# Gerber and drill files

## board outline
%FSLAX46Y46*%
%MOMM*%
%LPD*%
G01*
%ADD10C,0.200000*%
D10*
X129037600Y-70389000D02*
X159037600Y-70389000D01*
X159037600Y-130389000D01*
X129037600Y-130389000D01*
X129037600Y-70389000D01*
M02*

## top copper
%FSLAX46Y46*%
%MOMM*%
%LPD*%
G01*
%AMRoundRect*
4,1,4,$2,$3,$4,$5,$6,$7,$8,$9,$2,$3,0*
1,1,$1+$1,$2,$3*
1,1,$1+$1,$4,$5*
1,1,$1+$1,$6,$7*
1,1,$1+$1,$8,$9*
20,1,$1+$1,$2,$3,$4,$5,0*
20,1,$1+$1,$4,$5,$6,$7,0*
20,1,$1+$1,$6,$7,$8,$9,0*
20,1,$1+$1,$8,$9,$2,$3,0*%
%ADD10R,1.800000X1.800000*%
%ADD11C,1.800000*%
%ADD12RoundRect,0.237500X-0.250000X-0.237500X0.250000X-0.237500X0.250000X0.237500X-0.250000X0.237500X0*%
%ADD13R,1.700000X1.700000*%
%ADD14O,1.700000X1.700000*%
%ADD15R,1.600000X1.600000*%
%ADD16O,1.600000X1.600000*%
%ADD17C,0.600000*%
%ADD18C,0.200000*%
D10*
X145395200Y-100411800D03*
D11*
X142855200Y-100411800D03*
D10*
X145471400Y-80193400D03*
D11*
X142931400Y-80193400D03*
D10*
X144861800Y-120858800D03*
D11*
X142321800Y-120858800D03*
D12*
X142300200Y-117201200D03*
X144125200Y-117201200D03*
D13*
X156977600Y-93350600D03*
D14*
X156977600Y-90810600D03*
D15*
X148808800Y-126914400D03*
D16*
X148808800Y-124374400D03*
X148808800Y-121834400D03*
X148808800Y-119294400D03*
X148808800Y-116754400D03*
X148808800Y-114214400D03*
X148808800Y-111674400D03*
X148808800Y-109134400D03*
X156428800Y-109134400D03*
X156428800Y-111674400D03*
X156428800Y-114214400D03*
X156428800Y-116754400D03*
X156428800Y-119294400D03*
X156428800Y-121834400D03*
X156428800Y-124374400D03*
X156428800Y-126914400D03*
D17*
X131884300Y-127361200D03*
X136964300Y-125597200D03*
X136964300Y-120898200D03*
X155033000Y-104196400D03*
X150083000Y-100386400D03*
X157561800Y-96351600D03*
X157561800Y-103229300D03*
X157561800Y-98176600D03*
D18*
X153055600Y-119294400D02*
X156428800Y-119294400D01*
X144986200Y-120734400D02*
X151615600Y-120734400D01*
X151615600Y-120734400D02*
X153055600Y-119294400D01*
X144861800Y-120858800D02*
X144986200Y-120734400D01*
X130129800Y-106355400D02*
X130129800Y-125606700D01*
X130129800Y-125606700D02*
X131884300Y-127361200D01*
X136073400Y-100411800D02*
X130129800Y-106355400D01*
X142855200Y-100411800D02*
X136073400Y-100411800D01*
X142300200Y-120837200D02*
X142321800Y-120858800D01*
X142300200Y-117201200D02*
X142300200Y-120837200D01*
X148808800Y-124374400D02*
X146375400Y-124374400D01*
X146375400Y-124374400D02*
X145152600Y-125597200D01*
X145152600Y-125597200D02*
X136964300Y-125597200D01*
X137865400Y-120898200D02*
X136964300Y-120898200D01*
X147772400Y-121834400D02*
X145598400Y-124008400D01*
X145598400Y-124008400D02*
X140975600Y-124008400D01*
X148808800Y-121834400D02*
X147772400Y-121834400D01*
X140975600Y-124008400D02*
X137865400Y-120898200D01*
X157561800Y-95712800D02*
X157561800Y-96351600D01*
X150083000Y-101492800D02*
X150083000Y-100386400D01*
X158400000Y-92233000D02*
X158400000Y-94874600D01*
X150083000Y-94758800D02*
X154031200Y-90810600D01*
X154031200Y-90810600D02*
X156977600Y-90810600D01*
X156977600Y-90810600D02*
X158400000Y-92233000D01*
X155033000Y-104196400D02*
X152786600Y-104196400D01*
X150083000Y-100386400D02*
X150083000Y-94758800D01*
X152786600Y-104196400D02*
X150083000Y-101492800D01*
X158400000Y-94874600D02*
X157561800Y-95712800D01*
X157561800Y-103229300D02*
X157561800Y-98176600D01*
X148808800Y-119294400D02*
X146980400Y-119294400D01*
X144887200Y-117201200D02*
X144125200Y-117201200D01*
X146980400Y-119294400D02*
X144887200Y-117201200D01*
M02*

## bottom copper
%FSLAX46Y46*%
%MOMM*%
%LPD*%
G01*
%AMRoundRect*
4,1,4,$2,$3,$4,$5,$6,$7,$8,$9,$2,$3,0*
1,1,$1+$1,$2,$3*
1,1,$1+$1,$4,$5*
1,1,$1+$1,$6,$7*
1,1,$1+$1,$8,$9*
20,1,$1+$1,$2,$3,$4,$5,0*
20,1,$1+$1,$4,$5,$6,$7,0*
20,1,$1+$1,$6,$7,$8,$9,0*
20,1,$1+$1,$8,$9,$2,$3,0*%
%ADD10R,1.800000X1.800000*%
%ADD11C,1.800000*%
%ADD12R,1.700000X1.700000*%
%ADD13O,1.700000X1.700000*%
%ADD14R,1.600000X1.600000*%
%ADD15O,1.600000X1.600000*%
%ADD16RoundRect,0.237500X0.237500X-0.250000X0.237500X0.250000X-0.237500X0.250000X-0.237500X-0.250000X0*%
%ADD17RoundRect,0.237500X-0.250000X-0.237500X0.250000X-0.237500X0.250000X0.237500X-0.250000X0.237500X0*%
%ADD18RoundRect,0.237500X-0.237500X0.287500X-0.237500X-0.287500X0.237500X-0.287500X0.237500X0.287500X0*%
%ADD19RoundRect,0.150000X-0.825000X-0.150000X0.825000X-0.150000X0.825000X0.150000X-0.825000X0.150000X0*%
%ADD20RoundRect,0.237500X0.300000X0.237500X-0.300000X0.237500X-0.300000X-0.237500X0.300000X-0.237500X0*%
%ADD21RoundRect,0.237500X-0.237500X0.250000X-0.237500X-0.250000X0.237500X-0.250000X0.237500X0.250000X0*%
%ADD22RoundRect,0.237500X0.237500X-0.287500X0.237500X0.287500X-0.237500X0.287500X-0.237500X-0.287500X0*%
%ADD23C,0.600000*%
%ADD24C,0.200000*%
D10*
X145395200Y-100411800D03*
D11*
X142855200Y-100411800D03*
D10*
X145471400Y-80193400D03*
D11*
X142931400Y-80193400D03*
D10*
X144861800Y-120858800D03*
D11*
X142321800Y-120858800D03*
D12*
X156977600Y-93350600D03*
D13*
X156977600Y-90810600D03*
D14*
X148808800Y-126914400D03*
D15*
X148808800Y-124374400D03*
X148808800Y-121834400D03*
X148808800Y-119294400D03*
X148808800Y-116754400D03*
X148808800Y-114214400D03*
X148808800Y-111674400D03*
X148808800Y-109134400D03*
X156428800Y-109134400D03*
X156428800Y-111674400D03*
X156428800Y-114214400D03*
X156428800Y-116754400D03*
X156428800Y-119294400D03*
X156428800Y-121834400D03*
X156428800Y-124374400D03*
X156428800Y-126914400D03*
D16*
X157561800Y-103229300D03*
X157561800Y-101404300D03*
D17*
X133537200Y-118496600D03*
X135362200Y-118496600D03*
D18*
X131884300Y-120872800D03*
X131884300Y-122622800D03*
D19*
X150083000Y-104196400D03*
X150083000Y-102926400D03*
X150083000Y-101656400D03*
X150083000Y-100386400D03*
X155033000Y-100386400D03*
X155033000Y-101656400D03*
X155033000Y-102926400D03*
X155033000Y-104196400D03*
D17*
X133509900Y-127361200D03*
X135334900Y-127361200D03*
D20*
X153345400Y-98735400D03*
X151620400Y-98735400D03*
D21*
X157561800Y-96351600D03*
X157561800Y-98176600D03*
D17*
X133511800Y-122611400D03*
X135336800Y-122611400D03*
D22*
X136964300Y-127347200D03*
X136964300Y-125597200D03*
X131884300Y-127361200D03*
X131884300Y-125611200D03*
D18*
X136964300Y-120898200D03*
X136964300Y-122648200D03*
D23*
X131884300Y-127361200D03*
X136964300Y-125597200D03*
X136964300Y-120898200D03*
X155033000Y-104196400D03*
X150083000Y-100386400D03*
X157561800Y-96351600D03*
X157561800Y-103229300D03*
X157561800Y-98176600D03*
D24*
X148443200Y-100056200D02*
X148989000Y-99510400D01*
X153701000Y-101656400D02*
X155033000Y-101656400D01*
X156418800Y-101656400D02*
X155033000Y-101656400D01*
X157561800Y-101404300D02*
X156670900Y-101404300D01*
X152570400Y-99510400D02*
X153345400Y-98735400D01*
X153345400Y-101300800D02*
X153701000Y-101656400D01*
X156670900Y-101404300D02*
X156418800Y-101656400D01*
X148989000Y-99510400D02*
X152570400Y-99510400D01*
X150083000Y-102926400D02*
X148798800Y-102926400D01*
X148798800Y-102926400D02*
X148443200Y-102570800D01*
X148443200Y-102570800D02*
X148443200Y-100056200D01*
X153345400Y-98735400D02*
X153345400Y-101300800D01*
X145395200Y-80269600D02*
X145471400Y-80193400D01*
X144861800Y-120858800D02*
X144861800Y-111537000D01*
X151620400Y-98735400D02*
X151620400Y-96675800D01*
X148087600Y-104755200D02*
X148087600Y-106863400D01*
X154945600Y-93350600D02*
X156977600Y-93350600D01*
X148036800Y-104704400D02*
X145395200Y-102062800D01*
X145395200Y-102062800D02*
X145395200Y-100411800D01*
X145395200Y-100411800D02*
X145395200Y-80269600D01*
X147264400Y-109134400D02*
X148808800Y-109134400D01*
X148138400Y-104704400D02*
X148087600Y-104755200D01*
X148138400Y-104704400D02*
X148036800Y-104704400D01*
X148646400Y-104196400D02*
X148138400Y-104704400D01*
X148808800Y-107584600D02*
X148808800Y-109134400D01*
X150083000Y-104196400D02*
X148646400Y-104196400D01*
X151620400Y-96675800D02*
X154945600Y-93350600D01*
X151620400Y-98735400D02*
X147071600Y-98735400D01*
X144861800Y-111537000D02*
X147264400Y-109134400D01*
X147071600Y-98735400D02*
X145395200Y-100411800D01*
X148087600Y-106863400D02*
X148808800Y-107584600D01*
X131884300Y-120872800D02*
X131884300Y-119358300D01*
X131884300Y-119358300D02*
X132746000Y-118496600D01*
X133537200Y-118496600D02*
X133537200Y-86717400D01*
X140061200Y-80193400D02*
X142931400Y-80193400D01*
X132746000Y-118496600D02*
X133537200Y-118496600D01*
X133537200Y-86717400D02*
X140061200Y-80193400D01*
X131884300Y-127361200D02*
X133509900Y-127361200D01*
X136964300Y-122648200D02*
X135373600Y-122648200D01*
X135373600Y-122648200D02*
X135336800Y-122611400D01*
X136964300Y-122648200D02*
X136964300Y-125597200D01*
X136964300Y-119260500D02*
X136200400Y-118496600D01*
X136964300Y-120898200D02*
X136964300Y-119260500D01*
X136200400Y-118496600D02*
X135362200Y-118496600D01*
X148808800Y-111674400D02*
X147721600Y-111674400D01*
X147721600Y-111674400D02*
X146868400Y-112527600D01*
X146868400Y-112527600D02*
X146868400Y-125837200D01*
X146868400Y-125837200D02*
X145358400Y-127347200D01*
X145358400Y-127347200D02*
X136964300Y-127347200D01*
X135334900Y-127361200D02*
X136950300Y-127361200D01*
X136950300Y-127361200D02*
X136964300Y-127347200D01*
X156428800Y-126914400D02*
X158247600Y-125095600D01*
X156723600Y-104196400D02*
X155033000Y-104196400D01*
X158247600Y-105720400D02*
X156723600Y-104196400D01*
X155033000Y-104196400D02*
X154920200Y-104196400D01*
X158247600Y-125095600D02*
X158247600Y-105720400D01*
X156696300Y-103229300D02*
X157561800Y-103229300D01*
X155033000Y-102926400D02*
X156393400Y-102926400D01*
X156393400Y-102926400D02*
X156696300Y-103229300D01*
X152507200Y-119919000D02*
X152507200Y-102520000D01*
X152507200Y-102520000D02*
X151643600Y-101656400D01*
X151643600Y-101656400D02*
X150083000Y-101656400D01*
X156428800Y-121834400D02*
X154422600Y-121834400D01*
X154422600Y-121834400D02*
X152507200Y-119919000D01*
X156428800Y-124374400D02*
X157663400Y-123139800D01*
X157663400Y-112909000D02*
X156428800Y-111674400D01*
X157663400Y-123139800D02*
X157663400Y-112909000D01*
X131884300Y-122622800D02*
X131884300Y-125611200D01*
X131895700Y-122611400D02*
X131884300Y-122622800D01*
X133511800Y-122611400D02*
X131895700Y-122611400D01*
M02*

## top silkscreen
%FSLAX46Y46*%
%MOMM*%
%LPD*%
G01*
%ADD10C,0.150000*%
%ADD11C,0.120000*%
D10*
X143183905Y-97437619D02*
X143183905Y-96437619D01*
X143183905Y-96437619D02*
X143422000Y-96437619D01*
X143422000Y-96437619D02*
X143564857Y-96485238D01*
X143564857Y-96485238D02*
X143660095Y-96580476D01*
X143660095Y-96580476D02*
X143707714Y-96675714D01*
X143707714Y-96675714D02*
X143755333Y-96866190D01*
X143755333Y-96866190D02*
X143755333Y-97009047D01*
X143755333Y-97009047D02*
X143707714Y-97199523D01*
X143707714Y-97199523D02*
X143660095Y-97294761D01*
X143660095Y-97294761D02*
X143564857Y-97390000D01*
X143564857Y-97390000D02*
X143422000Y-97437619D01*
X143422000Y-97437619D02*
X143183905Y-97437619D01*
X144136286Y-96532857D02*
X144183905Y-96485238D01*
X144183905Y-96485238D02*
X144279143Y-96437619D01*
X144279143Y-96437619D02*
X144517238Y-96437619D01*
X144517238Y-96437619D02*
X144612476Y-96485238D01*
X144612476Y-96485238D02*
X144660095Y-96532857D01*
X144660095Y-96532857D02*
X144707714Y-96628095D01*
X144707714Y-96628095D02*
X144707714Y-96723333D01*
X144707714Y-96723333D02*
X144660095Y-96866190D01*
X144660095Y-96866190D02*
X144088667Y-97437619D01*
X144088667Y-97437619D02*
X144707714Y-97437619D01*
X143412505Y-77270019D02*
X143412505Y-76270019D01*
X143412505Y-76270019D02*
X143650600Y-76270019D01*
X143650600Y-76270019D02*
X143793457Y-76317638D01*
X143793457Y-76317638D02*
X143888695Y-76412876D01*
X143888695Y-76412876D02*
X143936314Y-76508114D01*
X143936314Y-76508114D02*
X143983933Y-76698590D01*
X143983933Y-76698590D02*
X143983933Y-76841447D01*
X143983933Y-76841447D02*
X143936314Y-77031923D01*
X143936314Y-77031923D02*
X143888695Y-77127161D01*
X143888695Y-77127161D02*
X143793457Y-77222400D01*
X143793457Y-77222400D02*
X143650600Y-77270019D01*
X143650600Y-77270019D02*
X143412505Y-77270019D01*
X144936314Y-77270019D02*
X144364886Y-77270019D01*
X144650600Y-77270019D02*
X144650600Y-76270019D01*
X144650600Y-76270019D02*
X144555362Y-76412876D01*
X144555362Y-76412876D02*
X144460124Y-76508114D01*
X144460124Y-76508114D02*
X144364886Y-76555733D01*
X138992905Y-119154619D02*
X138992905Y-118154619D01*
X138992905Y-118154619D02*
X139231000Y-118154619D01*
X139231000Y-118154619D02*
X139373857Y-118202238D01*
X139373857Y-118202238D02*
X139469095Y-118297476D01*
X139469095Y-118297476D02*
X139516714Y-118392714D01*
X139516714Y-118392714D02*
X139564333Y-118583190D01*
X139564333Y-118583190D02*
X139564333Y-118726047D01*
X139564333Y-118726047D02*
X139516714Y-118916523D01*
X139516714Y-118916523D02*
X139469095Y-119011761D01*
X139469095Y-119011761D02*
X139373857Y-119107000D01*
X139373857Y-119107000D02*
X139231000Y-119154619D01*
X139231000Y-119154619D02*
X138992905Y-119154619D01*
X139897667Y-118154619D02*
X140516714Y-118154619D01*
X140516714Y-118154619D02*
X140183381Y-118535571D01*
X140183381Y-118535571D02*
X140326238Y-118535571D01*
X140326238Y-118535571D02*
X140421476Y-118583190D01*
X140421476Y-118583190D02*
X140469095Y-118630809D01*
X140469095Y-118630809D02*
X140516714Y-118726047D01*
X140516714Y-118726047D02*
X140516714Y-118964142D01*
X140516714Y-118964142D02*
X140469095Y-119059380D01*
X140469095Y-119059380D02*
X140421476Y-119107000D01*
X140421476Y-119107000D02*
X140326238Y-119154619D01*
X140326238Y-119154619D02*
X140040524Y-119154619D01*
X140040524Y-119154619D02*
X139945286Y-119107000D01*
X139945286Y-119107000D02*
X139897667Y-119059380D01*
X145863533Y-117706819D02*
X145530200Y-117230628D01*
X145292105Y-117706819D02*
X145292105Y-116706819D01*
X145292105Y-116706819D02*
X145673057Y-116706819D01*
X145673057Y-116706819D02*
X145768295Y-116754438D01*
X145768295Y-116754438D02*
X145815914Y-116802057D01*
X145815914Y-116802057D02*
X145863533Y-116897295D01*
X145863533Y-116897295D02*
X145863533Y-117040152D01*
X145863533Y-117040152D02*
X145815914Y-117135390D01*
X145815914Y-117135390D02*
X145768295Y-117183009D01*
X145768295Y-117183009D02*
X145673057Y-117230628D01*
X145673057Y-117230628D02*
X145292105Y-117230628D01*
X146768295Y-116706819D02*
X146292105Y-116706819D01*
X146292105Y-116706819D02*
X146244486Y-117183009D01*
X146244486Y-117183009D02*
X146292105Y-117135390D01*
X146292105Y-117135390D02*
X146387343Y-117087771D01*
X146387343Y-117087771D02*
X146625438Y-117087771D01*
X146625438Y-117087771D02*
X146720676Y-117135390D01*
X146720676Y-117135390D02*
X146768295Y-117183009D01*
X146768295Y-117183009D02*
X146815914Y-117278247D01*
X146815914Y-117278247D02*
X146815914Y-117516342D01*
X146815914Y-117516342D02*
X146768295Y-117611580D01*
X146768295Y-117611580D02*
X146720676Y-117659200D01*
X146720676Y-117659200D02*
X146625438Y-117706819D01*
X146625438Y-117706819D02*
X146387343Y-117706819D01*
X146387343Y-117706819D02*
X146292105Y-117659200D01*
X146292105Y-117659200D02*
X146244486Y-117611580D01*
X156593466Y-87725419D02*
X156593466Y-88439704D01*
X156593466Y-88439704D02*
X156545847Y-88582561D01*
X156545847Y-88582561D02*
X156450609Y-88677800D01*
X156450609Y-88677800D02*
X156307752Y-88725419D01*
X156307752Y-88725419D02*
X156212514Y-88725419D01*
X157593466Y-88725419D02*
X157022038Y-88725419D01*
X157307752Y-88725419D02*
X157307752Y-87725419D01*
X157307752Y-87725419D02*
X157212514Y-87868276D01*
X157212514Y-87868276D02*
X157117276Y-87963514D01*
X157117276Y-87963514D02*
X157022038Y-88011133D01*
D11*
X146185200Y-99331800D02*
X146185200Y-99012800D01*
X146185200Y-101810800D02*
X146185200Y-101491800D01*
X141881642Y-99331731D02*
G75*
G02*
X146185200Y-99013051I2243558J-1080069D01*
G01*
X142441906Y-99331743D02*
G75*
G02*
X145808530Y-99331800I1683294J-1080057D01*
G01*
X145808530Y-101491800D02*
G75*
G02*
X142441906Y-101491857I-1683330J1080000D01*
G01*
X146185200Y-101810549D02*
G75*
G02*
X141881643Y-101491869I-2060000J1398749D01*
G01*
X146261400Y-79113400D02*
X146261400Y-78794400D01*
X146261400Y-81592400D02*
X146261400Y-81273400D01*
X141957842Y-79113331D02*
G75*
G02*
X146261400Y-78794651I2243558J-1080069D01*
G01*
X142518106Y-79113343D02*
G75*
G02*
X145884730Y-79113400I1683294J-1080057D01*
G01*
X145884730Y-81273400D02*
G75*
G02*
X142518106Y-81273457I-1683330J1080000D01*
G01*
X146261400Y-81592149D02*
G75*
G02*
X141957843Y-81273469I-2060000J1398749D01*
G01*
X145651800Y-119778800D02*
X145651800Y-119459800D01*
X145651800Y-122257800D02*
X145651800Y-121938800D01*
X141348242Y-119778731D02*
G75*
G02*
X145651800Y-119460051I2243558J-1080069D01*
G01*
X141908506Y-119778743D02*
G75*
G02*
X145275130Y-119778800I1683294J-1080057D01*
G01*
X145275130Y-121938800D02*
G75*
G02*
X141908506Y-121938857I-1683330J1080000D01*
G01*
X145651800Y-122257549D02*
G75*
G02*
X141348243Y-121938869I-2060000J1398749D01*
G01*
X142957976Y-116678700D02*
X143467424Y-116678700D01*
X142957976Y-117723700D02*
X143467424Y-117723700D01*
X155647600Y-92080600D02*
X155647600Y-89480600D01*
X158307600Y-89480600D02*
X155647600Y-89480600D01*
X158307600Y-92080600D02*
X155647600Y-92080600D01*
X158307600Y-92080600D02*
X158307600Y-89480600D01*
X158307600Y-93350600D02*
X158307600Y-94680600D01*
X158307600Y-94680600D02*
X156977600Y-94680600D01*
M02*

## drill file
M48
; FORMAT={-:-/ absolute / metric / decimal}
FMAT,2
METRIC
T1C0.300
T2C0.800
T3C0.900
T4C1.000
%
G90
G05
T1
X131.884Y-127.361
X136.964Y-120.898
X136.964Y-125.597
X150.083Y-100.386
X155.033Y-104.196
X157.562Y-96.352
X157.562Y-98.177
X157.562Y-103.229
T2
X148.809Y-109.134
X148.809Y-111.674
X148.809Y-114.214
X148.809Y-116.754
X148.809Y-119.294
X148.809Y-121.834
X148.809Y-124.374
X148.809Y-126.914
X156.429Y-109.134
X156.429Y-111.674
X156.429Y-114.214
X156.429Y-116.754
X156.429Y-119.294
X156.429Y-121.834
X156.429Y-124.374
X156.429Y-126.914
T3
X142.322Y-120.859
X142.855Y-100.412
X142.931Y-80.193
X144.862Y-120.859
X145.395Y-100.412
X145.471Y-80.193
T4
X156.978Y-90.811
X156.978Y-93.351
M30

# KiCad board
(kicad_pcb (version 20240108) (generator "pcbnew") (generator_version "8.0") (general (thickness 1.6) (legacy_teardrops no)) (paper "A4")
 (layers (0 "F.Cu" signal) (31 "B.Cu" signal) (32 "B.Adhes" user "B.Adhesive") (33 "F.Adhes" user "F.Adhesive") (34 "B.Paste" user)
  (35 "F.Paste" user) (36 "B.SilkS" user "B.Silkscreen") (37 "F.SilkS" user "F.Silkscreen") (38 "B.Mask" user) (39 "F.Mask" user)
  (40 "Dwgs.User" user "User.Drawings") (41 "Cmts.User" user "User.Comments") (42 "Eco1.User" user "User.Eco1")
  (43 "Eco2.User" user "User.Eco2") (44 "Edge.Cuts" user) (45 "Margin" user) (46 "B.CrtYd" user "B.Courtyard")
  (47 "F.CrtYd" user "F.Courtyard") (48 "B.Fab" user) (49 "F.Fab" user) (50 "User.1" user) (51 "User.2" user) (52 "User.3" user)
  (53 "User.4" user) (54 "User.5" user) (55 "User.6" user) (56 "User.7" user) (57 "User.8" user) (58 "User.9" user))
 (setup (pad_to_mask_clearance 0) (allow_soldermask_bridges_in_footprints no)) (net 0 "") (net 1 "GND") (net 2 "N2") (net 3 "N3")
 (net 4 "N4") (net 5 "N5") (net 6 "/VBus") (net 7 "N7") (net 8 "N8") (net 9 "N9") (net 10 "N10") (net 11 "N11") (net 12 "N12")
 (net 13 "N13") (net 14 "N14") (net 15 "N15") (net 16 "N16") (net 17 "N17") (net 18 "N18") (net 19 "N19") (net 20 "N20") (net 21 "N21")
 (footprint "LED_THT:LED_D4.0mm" (layer "F.Cu") (at 145.3952 100.4118 180)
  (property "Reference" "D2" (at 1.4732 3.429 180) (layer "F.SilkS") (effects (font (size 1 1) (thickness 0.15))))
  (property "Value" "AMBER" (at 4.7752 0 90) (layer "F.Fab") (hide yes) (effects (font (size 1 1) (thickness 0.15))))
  (fp_line (start -0.79 1.08) (end -0.79 1.399) (stroke (width 0.12) (type solid)) (layer "F.SilkS"))
  (fp_line (start -0.79 -1.399) (end -0.79 -1.08) (stroke (width 0.12) (type solid)) (layer "F.SilkS"))
  (fp_arc (start 3.513558 1.080069) (mid 1.453882 2.483201) (end -0.79 1.398749) (stroke (width 0.12) (type solid)) (layer "F.SilkS"))
  (fp_arc (start 2.953294 1.080057) (mid 1.269966 2) (end -0.41333 1.08) (stroke (width 0.12) (type solid)) (layer "F.SilkS"))
  (fp_arc (start -0.41333 -1.08) (mid 1.269966 -2) (end 2.953294 -1.080057) (stroke (width 0.12) (type solid)) (layer "F.SilkS"))
  (fp_arc (start -0.79 -1.398749) (mid 1.453882 -2.483201) (end 3.513558 -1.080069) (stroke (width 0.12) (type solid)) (layer "F.SilkS"))
  (pad "1" thru_hole rect (at 0 0 180) (size 1.8 1.8) (drill 0.9) (layers "*.Cu" "*.Mask") (remove_unused_layers no) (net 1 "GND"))
  (pad "2" thru_hole circle (at 2.54 0 180) (size 1.8 1.8) (drill 0.9) (layers "*.Cu" "*.Mask") (remove_unused_layers no) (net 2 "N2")))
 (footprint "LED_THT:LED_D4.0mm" (layer "F.Cu") (at 145.4714 80.1934 180)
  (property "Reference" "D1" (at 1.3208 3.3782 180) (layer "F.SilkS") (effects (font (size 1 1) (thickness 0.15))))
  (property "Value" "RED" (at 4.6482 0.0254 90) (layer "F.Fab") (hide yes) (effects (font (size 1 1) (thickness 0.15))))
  (fp_line (start -0.79 1.08) (end -0.79 1.399) (stroke (width 0.12) (type solid)) (layer "F.SilkS"))
  (fp_line (start -0.79 -1.399) (end -0.79 -1.08) (stroke (width 0.12) (type solid)) (layer "F.SilkS"))
  (fp_arc (start 3.513558 1.080069) (mid 1.453882 2.483201) (end -0.79 1.398749) (stroke (width 0.12) (type solid)) (layer "F.SilkS"))
  (fp_arc (start 2.953294 1.080057) (mid 1.269966 2) (end -0.41333 1.08) (stroke (width 0.12) (type solid)) (layer "F.SilkS"))
  (fp_arc (start -0.41333 -1.08) (mid 1.269966 -2) (end 2.953294 -1.080057) (stroke (width 0.12) (type solid)) (layer "F.SilkS"))
  (fp_arc (start -0.79 -1.398749) (mid 1.453882 -2.483201) (end 3.513558 -1.080069) (stroke (width 0.12) (type solid)) (layer "F.SilkS"))
  (pad "1" thru_hole rect (at 0 0 180) (size 1.8 1.8) (drill 0.9) (layers "*.Cu" "*.Mask") (remove_unused_layers no) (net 1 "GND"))
  (pad "2" thru_hole circle (at 2.54 0 180) (size 1.8 1.8) (drill 0.9) (layers "*.Cu" "*.Mask") (remove_unused_layers no) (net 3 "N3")))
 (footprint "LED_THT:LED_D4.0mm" (layer "F.Cu") (at 144.8618 120.8588 180)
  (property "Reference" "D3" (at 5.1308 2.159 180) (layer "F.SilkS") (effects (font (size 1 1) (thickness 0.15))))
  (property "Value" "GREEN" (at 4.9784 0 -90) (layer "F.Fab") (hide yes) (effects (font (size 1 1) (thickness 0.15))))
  (fp_line (start -0.79 1.08) (end -0.79 1.399) (stroke (width 0.12) (type solid)) (layer "F.SilkS"))
  (fp_line (start -0.79 -1.399) (end -0.79 -1.08) (stroke (width 0.12) (type solid)) (layer "F.SilkS"))
  (fp_arc (start 3.513558 1.080069) (mid 1.453882 2.483201) (end -0.79 1.398749) (stroke (width 0.12) (type solid)) (layer "F.SilkS"))
  (fp_arc (start 2.953294 1.080057) (mid 1.269966 2) (end -0.41333 1.08) (stroke (width 0.12) (type solid)) (layer "F.SilkS"))
  (fp_arc (start -0.41333 -1.08) (mid 1.269966 -2) (end 2.953294 -1.080057) (stroke (width 0.12) (type solid)) (layer "F.SilkS"))
  (fp_arc (start -0.79 -1.398749) (mid 1.453882 -2.483201) (end 3.513558 -1.080069) (stroke (width 0.12) (type solid)) (layer "F.SilkS"))
  (pad "1" thru_hole rect (at 0 0 180) (size 1.8 1.8) (drill 0.9) (layers "*.Cu" "*.Mask") (remove_unused_layers no) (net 1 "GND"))
  (pad "2" thru_hole circle (at 2.54 0 180) (size 1.8 1.8) (drill 0.9) (layers "*.Cu" "*.Mask") (remove_unused_layers no) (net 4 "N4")))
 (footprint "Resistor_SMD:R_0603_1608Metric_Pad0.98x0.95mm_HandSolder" (layer "F.Cu") (at 143.2127 117.2012)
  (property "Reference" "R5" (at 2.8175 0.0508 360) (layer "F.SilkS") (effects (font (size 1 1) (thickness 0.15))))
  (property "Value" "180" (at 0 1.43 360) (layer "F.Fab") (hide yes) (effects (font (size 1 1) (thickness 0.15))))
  (fp_line (start -0.254724 -0.5225) (end 0.254724 -0.5225) (stroke (width 0.12) (type solid)) (layer "F.SilkS"))
  (fp_line (start -0.254724 0.5225) (end 0.254724 0.5225) (stroke (width 0.12) (type solid)) (layer "F.SilkS"))
  (pad "1" smd roundrect (at -0.9125 0) (size 0.975 0.95) (layers "F.Cu" "F.Paste" "F.Mask") (roundrect_rratio 0.25) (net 4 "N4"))
  (pad "2" smd roundrect (at 0.9125 0) (size 0.975 0.95) (layers "F.Cu" "F.Paste" "F.Mask") (roundrect_rratio 0.25) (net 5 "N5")))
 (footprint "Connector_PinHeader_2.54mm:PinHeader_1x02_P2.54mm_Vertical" (layer "F.Cu") (at 156.9776 93.3506 180)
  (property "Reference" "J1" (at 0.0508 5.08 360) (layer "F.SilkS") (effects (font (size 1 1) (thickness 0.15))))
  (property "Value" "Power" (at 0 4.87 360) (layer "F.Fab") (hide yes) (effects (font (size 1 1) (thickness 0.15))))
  (fp_line (start 1.33 1.27) (end 1.33 3.87) (stroke (width 0.12) (type solid)) (layer "F.SilkS"))
  (fp_line (start -1.33 3.87) (end 1.33 3.87) (stroke (width 0.12) (type solid)) (layer "F.SilkS"))
  (fp_line (start -1.33 1.27) (end 1.33 1.27) (stroke (width 0.12) (type solid)) (layer "F.SilkS"))
  (fp_line (start -1.33 1.27) (end -1.33 3.87) (stroke (width 0.12) (type solid)) (layer "F.SilkS"))
  (fp_line (start -1.33 0) (end -1.33 -1.33) (stroke (width 0.12) (type solid)) (layer "F.SilkS"))
  (fp_line (start -1.33 -1.33) (end 0 -1.33) (stroke (width 0.12) (type solid)) (layer "F.SilkS"))
  (pad "1" thru_hole rect (at 0 0 180) (size 1.7 1.7) (drill 1) (layers "*.Cu" "*.Mask") (remove_unused_layers no) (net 1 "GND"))
  (pad "2" thru_hole oval (at 0 2.54 180) (size 1.7 1.7) (drill 1) (layers "*.Cu" "*.Mask") (remove_unused_layers no) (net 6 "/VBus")))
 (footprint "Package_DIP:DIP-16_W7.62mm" (layer "B.Cu") (at 148.8088 126.9144)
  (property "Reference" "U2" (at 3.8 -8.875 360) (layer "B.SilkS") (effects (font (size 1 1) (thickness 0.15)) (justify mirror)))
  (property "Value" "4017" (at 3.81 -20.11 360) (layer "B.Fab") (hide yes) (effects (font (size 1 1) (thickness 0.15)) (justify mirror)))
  (pad "1" thru_hole rect (at 0 0) (size 1.6 1.6) (drill 0.8) (layers "*.Cu" "*.Mask") (remove_unused_layers no) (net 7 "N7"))
  (pad "2" thru_hole oval (at 0 -2.54) (size 1.6 1.6) (drill 0.8) (layers "*.Cu" "*.Mask") (remove_unused_layers no) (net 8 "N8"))
  (pad "3" thru_hole oval (at 0 -5.08) (size 1.6 1.6) (drill 0.8) (layers "*.Cu" "*.Mask") (remove_unused_layers no) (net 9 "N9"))
  (pad "4" thru_hole oval (at 0 -7.62) (size 1.6 1.6) (drill 0.8) (layers "*.Cu" "*.Mask") (remove_unused_layers no) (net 5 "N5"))
  (pad "5" thru_hole oval (at 0 -10.16) (size 1.6 1.6) (drill 0.8) (layers "*.Cu" "*.Mask") (remove_unused_layers no) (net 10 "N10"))
  (pad "6" thru_hole oval (at 0 -12.7) (size 1.6 1.6) (drill 0.8) (layers "*.Cu" "*.Mask") (remove_unused_layers no) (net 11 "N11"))
  (pad "7" thru_hole oval (at 0 -15.24) (size 1.6 1.6) (drill 0.8) (layers "*.Cu" "*.Mask") (remove_unused_layers no) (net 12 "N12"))
  (pad "8" thru_hole oval (at 0 -17.78) (size 1.6 1.6) (drill 0.8) (layers "*.Cu" "*.Mask") (remove_unused_layers no) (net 1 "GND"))
  (pad "9" thru_hole oval (at 7.62 -17.78) (size 1.6 1.6) (drill 0.8) (layers "*.Cu" "*.Mask") (remove_unused_layers no) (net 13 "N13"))
  (pad "10" thru_hole oval (at 7.62 -15.24) (size 1.6 1.6) (drill 0.8) (layers "*.Cu" "*.Mask") (remove_unused_layers no) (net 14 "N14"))
  (pad "11" thru_hole oval (at 7.62 -12.7) (size 1.6 1.6) (drill 0.8) (layers "*.Cu" "*.Mask") (remove_unused_layers no) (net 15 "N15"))
  (pad "12" thru_hole oval (at 7.62 -10.16) (size 1.6 1.6) (drill 0.8) (layers "*.Cu" "*.Mask") (remove_unused_layers no) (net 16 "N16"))
  (pad "13" thru_hole oval (at 7.62 -7.62) (size 1.6 1.6) (drill 0.8) (layers "*.Cu" "*.Mask") (remove_unused_layers no) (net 1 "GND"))
  (pad "14" thru_hole oval (at 7.62 -5.08) (size 1.6 1.6) (drill 0.8) (layers "*.Cu" "*.Mask") (remove_unused_layers no) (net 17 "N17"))
  (pad "15" thru_hole oval (at 7.62 -2.54) (size 1.6 1.6) (drill 0.8) (layers "*.Cu" "*.Mask") (remove_unused_layers no) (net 14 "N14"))
  (pad "16" thru_hole oval (at 7.62 0) (size 1.6 1.6) (drill 0.8) (layers "*.Cu" "*.Mask") (remove_unused_layers no) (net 6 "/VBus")))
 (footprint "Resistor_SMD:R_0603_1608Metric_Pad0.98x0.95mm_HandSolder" (layer "B.Cu") (at 157.5618 102.3168 90)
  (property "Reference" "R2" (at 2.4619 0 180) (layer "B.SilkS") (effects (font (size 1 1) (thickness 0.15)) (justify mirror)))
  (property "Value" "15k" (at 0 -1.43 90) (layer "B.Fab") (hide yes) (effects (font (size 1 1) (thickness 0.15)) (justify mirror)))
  (pad "1" smd roundrect (at -0.9125 0 90) (size 0.975 0.95) (layers "B.Cu" "B.Paste" "B.Mask") (roundrect_rratio 0.25) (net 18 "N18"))
  (pad "2" smd roundrect (at 0.9125 0 90) (size 0.975 0.95) (layers "B.Cu" "B.Paste" "B.Mask") (roundrect_rratio 0.25) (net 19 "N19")))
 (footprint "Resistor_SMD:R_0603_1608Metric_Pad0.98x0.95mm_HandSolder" (layer "B.Cu") (at 134.4497 118.4966)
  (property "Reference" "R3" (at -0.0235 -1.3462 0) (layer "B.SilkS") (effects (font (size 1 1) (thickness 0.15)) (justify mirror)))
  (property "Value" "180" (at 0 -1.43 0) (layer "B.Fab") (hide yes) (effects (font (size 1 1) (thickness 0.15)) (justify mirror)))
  (pad "1" smd roundrect (at -0.9125 0) (size 0.975 0.95) (layers "B.Cu" "B.Paste" "B.Mask") (roundrect_rratio 0.25) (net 3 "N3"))
  (pad "2" smd roundrect (at 0.9125 0) (size 0.975 0.95) (layers "B.Cu" "B.Paste" "B.Mask") (roundrect_rratio 0.25) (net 9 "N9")))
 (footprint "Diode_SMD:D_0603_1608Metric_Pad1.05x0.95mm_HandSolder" (layer "B.Cu") (at 131.8843 121.7478 -90)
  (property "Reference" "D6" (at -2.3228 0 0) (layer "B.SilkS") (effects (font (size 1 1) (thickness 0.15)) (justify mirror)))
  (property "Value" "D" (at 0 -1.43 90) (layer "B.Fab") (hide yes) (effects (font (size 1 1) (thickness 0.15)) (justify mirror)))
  (pad "1" smd roundrect (at -0.875 0 270) (size 1.05 0.95) (layers "B.Cu" "B.Paste" "B.Mask") (roundrect_rratio 0.25) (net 3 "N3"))
  (pad "2" smd roundrect (at 0.875 0 270) (size 1.05 0.95) (layers "B.Cu" "B.Paste" "B.Mask") (roundrect_rratio 0.25) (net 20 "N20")))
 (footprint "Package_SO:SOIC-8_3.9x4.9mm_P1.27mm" (layer "B.Cu") (at 152.558 102.2914)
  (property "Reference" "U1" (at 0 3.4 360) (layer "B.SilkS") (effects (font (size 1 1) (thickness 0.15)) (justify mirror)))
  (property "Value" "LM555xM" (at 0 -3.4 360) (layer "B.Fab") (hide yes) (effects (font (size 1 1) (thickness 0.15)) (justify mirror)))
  (pad "1" smd roundrect (at -2.475 1.905) (size 1.95 0.6) (layers "B.Cu" "B.Paste" "B.Mask") (roundrect_rratio 0.25) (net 1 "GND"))
  (pad "2" smd roundrect (at -2.475 0.635) (size 1.95 0.6) (layers "B.Cu" "B.Paste" "B.Mask") (roundrect_rratio 0.25) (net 19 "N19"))
  (pad "3" smd roundrect (at -2.475 -0.635) (size 1.95 0.6) (layers "B.Cu" "B.Paste" "B.Mask") (roundrect_rratio 0.25) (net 17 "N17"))
  (pad "4" smd roundrect (at -2.475 -1.905) (size 1.95 0.6) (layers "B.Cu" "B.Paste" "B.Mask") (roundrect_rratio 0.25) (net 6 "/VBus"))
  (pad "5" smd roundrect (at 2.475 -1.905) (size 1.95 0.6) (layers "B.Cu" "B.Paste" "B.Mask") (roundrect_rratio 0.25) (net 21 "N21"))
  (pad "6" smd roundrect (at 2.475 -0.635) (size 1.95 0.6) (layers "B.Cu" "B.Paste" "B.Mask") (roundrect_rratio 0.25) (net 19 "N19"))
  (pad "7" smd roundrect (at 2.475 0.635) (size 1.95 0.6) (layers "B.Cu" "B.Paste" "B.Mask") (roundrect_rratio 0.25) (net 18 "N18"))
  (pad "8" smd roundrect (at 2.475 1.905) (size 1.95 0.6) (layers "B.Cu" "B.Paste" "B.Mask") (roundrect_rratio 0.25) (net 6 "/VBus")))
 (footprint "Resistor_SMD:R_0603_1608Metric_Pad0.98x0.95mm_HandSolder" (layer "B.Cu") (at 134.4224 127.3612)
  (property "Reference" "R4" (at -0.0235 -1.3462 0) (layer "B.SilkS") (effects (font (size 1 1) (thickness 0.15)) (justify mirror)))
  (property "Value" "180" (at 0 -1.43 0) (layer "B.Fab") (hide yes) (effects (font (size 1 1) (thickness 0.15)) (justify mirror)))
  (pad "1" smd roundrect (at -0.9125 0) (size 0.975 0.95) (layers "B.Cu" "B.Paste" "B.Mask") (roundrect_rratio 0.25) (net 2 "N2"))
  (pad "2" smd roundrect (at 0.9125 0) (size 0.975 0.95) (layers "B.Cu" "B.Paste" "B.Mask") (roundrect_rratio 0.25) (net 12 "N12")))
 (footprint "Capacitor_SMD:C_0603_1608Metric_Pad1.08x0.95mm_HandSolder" (layer "B.Cu") (at 152.4829 98.7354 180)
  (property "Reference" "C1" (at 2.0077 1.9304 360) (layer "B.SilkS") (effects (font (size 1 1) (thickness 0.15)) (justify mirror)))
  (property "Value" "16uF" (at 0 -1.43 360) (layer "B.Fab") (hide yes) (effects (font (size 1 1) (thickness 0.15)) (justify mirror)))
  (pad "1" smd roundrect (at -0.8625 0 180) (size 1.075 0.95) (layers "B.Cu" "B.Paste" "B.Mask") (roundrect_rratio 0.25) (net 19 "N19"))
  (pad "2" smd roundrect (at 0.8625 0 180) (size 1.075 0.95) (layers "B.Cu" "B.Paste" "B.Mask") (roundrect_rratio 0.25) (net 1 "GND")))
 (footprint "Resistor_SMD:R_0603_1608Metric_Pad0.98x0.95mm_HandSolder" (layer "B.Cu") (at 157.5618 97.2641 -90)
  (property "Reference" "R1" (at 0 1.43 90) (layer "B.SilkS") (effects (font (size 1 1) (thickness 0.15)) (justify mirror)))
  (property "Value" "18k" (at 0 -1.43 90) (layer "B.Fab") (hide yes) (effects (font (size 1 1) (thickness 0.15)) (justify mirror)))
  (pad "1" smd roundrect (at -0.9125 0 270) (size 0.975 0.95) (layers "B.Cu" "B.Paste" "B.Mask") (roundrect_rratio 0.25) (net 6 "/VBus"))
  (pad "2" smd roundrect (at 0.9125 0 270) (size 0.975 0.95) (layers "B.Cu" "B.Paste" "B.Mask") (roundrect_rratio 0.25) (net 18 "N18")))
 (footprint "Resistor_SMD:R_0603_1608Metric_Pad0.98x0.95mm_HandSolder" (layer "B.Cu") (at 134.4243 122.6114)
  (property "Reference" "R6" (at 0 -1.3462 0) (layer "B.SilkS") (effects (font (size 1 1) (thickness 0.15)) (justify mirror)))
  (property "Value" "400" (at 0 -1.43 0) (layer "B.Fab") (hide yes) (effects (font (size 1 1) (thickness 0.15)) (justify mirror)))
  (pad "1" smd roundrect (at -0.9125 0) (size 0.975 0.95) (layers "B.Cu" "B.Paste" "B.Mask") (roundrect_rratio 0.25) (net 20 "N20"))
  (pad "2" smd roundrect (at 0.9125 0) (size 0.975 0.95) (layers "B.Cu" "B.Paste" "B.Mask") (roundrect_rratio 0.25) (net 8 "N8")))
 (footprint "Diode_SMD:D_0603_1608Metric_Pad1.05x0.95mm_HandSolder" (layer "B.Cu") (at 136.9643 126.4722 90)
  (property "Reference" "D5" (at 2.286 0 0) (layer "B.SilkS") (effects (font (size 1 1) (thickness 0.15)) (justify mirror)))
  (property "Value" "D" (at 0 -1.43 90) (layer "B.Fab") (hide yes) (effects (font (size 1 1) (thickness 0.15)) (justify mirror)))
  (pad "1" smd roundrect (at -0.875 0 90) (size 1.05 0.95) (layers "B.Cu" "B.Paste" "B.Mask") (roundrect_rratio 0.25) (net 12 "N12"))
  (pad "2" smd roundrect (at 0.875 0 90) (size 1.05 0.95) (layers "B.Cu" "B.Paste" "B.Mask") (roundrect_rratio 0.25) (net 8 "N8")))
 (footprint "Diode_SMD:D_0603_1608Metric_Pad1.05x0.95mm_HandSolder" (layer "B.Cu") (at 131.8843 126.4862 90)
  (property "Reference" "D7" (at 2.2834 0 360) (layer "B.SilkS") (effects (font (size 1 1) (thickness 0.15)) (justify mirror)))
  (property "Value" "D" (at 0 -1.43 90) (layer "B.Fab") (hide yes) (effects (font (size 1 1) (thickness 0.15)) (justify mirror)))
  (pad "1" smd roundrect (at -0.875 0 90) (size 1.05 0.95) (layers "B.Cu" "B.Paste" "B.Mask") (roundrect_rratio 0.25) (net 2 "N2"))
  (pad "2" smd roundrect (at 0.875 0 90) (size 1.05 0.95) (layers "B.Cu" "B.Paste" "B.Mask") (roundrect_rratio 0.25) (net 20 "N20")))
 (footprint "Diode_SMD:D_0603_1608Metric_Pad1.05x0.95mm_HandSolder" (layer "B.Cu") (at 136.9643 121.7732 -90)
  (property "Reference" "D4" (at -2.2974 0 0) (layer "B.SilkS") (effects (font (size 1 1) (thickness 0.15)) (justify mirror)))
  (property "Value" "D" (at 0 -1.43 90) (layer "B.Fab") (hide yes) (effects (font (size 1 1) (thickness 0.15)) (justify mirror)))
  (pad "1" smd roundrect (at -0.875 0 270) (size 1.05 0.95) (layers "B.Cu" "B.Paste" "B.Mask") (roundrect_rratio 0.25) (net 9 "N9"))
  (pad "2" smd roundrect (at 0.875 0 270) (size 1.05 0.95) (layers "B.Cu" "B.Paste" "B.Mask") (roundrect_rratio 0.25) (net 8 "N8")))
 (gr_rect (start 129.0376 70.389) (end 159.0376 130.389) (stroke (width 0.2) (type default)) (fill none) (layer "Edge.Cuts"))
 (segment (start 148.4432 100.0562) (end 148.989 99.5104) (width 0.2) (layer "B.Cu") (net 19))
 (segment (start 153.701 101.6564) (end 155.033 101.6564) (width 0.2) (layer "B.Cu") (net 19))
 (segment (start 156.4188 101.6564) (end 155.033 101.6564) (width 0.2) (layer "B.Cu") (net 19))
 (segment (start 157.5618 101.4043) (end 156.6709 101.4043) (width 0.2) (layer "B.Cu") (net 19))
 (segment (start 152.5704 99.5104) (end 153.3454 98.7354) (width 0.2) (layer "B.Cu") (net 19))
 (segment (start 153.3454 101.3008) (end 153.701 101.6564) (width 0.2) (layer "B.Cu") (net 19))
 (segment (start 156.6709 101.4043) (end 156.4188 101.6564) (width 0.2) (layer "B.Cu") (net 19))
 (segment (start 148.989 99.5104) (end 152.5704 99.5104) (width 0.2) (layer "B.Cu") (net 19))
 (segment (start 150.083 102.9264) (end 148.7988 102.9264) (width 0.2) (layer "B.Cu") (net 19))
 (segment (start 148.7988 102.9264) (end 148.4432 102.5708) (width 0.2) (layer "B.Cu") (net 19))
 (segment (start 148.4432 102.5708) (end 148.4432 100.0562) (width 0.2) (layer "B.Cu") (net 19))
 (segment (start 153.3454 98.7354) (end 153.3454 101.3008) (width 0.2) (layer "B.Cu") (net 19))
 (segment (start 153.0556 119.2944) (end 156.4288 119.2944) (width 0.2) (layer "F.Cu") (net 1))
 (segment (start 144.9862 120.7344) (end 151.6156 120.7344) (width 0.2) (layer "F.Cu") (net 1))
 (segment (start 151.6156 120.7344) (end 153.0556 119.2944) (width 0.2) (layer "F.Cu") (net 1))
 (segment (start 144.8618 120.8588) (end 144.9862 120.7344) (width 0.2) (layer "F.Cu") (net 1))
 (segment (start 145.3952 80.2696) (end 145.4714 80.1934) (width 0.2) (layer "B.Cu") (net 1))
 (segment (start 144.8618 120.8588) (end 144.8618 111.537) (width 0.2) (layer "B.Cu") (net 1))
 (segment (start 151.6204 98.7354) (end 151.6204 96.6758) (width 0.2) (layer "B.Cu") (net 1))
 (segment (start 148.0876 104.7552) (end 148.0876 106.8634) (width 0.2) (layer "B.Cu") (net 1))
 (segment (start 154.9456 93.3506) (end 156.9776 93.3506) (width 0.2) (layer "B.Cu") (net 1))
 (segment (start 148.0368 104.7044) (end 145.3952 102.0628) (width 0.2) (layer "B.Cu") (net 1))
 (segment (start 145.3952 102.0628) (end 145.3952 100.4118) (width 0.2) (layer "B.Cu") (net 1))
 (segment (start 145.3952 100.4118) (end 145.3952 80.2696) (width 0.2) (layer "B.Cu") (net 1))
 (segment (start 147.2644 109.1344) (end 148.8088 109.1344) (width 0.2) (layer "B.Cu") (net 1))
 (segment (start 148.1384 104.7044) (end 148.0876 104.7552) (width 0.2) (layer "B.Cu") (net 1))
 (segment (start 148.1384 104.7044) (end 148.0368 104.7044) (width 0.2) (layer "B.Cu") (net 1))
 (segment (start 148.6464 104.1964) (end 148.1384 104.7044) (width 0.2) (layer "B.Cu") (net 1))
 (segment (start 148.8088 107.5846) (end 148.8088 109.1344) (width 0.2) (layer "B.Cu") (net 1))
 (segment (start 150.083 104.1964) (end 148.6464 104.1964) (width 0.2) (layer "B.Cu") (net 1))
 (segment (start 151.6204 96.6758) (end 154.9456 93.3506) (width 0.2) (layer "B.Cu") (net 1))
 (segment (start 151.6204 98.7354) (end 147.0716 98.7354) (width 0.2) (layer "B.Cu") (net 1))
 (segment (start 144.8618 111.537) (end 147.2644 109.1344) (width 0.2) (layer "B.Cu") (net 1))
 (segment (start 147.0716 98.7354) (end 145.3952 100.4118) (width 0.2) (layer "B.Cu") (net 1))
 (segment (start 148.0876 106.8634) (end 148.8088 107.5846) (width 0.2) (layer "B.Cu") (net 1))
 (segment (start 131.8843 120.8728) (end 131.8843 119.3583) (width 0.2) (layer "B.Cu") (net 3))
 (segment (start 131.8843 119.3583) (end 132.746 118.4966) (width 0.2) (layer "B.Cu") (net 3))
 (segment (start 133.5372 118.4966) (end 133.5372 86.7174) (width 0.2) (layer "B.Cu") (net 3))
 (segment (start 140.0612 80.1934) (end 142.9314 80.1934) (width 0.2) (layer "B.Cu") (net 3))
 (segment (start 132.746 118.4966) (end 133.5372 118.4966) (width 0.2) (layer "B.Cu") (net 3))
 (segment (start 133.5372 86.7174) (end 140.0612 80.1934) (width 0.2) (layer "B.Cu") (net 3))
 (segment (start 130.1298 106.3554) (end 130.1298 125.6067) (width 0.2) (layer "F.Cu") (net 2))
 (segment (start 130.1298 125.6067) (end 131.8843 127.3612) (width 0.2) (layer "F.Cu") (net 2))
 (segment (start 136.0734 100.4118) (end 130.1298 106.3554) (width 0.2) (layer "F.Cu") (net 2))
 (segment (start 142.8552 100.4118) (end 136.0734 100.4118) (width 0.2) (layer "F.Cu") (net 2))
 (via (at 131.8843 127.3612) (size 0.6) (drill 0.3) (layers "F.Cu" "B.Cu") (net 2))
 (segment (start 131.8843 127.3612) (end 133.5099 127.3612) (width 0.2) (layer "B.Cu") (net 2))
 (segment (start 142.3002 120.8372) (end 142.3218 120.8588) (width 0.2) (layer "F.Cu") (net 4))
 (segment (start 142.3002 117.2012) (end 142.3002 120.8372) (width 0.2) (layer "F.Cu") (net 4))
 (segment (start 148.8088 124.3744) (end 146.3754 124.3744) (width 0.2) (layer "F.Cu") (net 8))
 (segment (start 146.3754 124.3744) (end 145.1526 125.5972) (width 0.2) (layer "F.Cu") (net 8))
 (segment (start 145.1526 125.5972) (end 136.9643 125.5972) (width 0.2) (layer "F.Cu") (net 8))
 (via (at 136.9643 125.5972) (size 0.6) (drill 0.3) (layers "F.Cu" "B.Cu") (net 8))
 (segment (start 136.9643 122.6482) (end 135.3736 122.6482) (width 0.2) (layer "B.Cu") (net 8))
 (segment (start 135.3736 122.6482) (end 135.3368 122.6114) (width 0.2) (layer "B.Cu") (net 8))
 (segment (start 136.9643 122.6482) (end 136.9643 125.5972) (width 0.2) (layer "B.Cu") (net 8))
 (segment (start 137.8654 120.8982) (end 136.9643 120.8982) (width 0.2) (layer "F.Cu") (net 9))
 (segment (start 147.7724 121.8344) (end 145.5984 124.0084) (width 0.2) (layer "F.Cu") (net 9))
 (segment (start 145.5984 124.0084) (end 140.9756 124.0084) (width 0.2) (layer "F.Cu") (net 9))
 (segment (start 148.8088 121.8344) (end 147.7724 121.8344) (width 0.2) (layer "F.Cu") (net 9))
 (segment (start 140.9756 124.0084) (end 137.8654 120.8982) (width 0.2) (layer "F.Cu") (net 9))
 (via (at 136.9643 120.8982) (size 0.6) (drill 0.3) (layers "F.Cu" "B.Cu") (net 9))
 (segment (start 136.9643 119.2605) (end 136.2004 118.4966) (width 0.2) (layer "B.Cu") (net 9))
 (segment (start 136.9643 120.8982) (end 136.9643 119.2605) (width 0.2) (layer "B.Cu") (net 9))
 (segment (start 136.2004 118.4966) (end 135.3622 118.4966) (width 0.2) (layer "B.Cu") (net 9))
 (segment (start 148.8088 111.6744) (end 147.7216 111.6744) (width 0.2) (layer "B.Cu") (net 12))
 (segment (start 147.7216 111.6744) (end 146.8684 112.5276) (width 0.2) (layer "B.Cu") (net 12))
 (segment (start 146.8684 112.5276) (end 146.8684 125.8372) (width 0.2) (layer "B.Cu") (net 12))
 (segment (start 146.8684 125.8372) (end 145.3584 127.3472) (width 0.2) (layer "B.Cu") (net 12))
 (segment (start 145.3584 127.3472) (end 136.9643 127.3472) (width 0.2) (layer "B.Cu") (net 12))
 (segment (start 135.3349 127.3612) (end 136.9503 127.3612) (width 0.2) (layer "B.Cu") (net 12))
 (segment (start 136.9503 127.3612) (end 136.9643 127.3472) (width 0.2) (layer "B.Cu") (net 12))
 (segment (start 157.5618 95.7128) (end 157.5618 96.3516) (width 0.2) (layer "F.Cu") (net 6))
 (segment (start 150.083 101.4928) (end 150.083 100.3864) (width 0.2) (layer "F.Cu") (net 6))
 (segment (start 158.4 92.233) (end 158.4 94.8746) (width 0.2) (layer "F.Cu") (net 6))
 (segment (start 150.083 94.7588) (end 154.0312 90.8106) (width 0.2) (layer "F.Cu") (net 6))
 (segment (start 154.0312 90.8106) (end 156.9776 90.8106) (width 0.2) (layer "F.Cu") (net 6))
 (segment (start 156.9776 90.8106) (end 158.4 92.233) (width 0.2) (layer "F.Cu") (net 6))
 (segment (start 155.033 104.1964) (end 152.7866 104.1964) (width 0.2) (layer "F.Cu") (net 6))
 (segment (start 150.083 100.3864) (end 150.083 94.7588) (width 0.2) (layer "F.Cu") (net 6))
 (segment (start 152.7866 104.1964) (end 150.083 101.4928) (width 0.2) (layer "F.Cu") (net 6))
 (segment (start 158.4 94.8746) (end 157.5618 95.7128) (width 0.2) (layer "F.Cu") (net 6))
 (via (at 155.033 104.1964) (size 0.6) (drill 0.3) (layers "F.Cu" "B.Cu") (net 6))
 (via (at 150.083 100.3864) (size 0.6) (drill 0.3) (layers "F.Cu" "B.Cu") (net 6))
 (via (at 157.5618 96.3516) (size 0.6) (drill 0.3) (layers "F.Cu" "B.Cu") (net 6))
 (segment (start 156.4288 126.9144) (end 158.2476 125.0956) (width 0.2) (layer "B.Cu") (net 6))
 (segment (start 156.7236 104.1964) (end 155.033 104.1964) (width 0.2) (layer "B.Cu") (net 6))
 (segment (start 158.2476 105.7204) (end 156.7236 104.1964) (width 0.2) (layer "B.Cu") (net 6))
 (segment (start 155.033 104.1964) (end 154.9202 104.1964) (width 0.2) (layer "B.Cu") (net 6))
 (segment (start 158.2476 125.0956) (end 158.2476 105.7204) (width 0.2) (layer "B.Cu") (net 6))
 (segment (start 157.5618 103.2293) (end 157.5618 98.1766) (width 0.2) (layer "F.Cu") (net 18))
 (via (at 157.5618 103.2293) (size 0.6) (drill 0.3) (layers "F.Cu" "B.Cu") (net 18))
 (via (at 157.5618 98.1766) (size 0.6) (drill 0.3) (layers "F.Cu" "B.Cu") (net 18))
 (segment (start 156.6963 103.2293) (end 157.5618 103.2293) (width 0.2) (layer "B.Cu") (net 18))
 (segment (start 155.033 102.9264) (end 156.3934 102.9264) (width 0.2) (layer "B.Cu") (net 18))
 (segment (start 156.3934 102.9264) (end 156.6963 103.2293) (width 0.2) (layer "B.Cu") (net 18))
 (segment (start 148.8088 119.2944) (end 146.9804 119.2944) (width 0.2) (layer "F.Cu") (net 5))
 (segment (start 144.8872 117.2012) (end 144.1252 117.2012) (width 0.2) (layer "F.Cu") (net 5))
 (segment (start 146.9804 119.2944) (end 144.8872 117.2012) (width 0.2) (layer "F.Cu") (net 5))
 (segment (start 152.5072 119.919) (end 152.5072 102.52) (width 0.2) (layer "B.Cu") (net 17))
 (segment (start 152.5072 102.52) (end 151.6436 101.6564) (width 0.2) (layer "B.Cu") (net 17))
 (segment (start 151.6436 101.6564) (end 150.083 101.6564) (width 0.2) (layer "B.Cu") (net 17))
 (segment (start 156.4288 121.8344) (end 154.4226 121.8344) (width 0.2) (layer "B.Cu") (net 17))
 (segment (start 154.4226 121.8344) (end 152.5072 119.919) (width 0.2) (layer "B.Cu") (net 17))
 (segment (start 156.4288 124.3744) (end 157.6634 123.1398) (width 0.2) (layer "B.Cu") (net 14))
 (segment (start 157.6634 112.909) (end 156.4288 111.6744) (width 0.2) (layer "B.Cu") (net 14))
 (segment (start 157.6634 123.1398) (end 157.6634 112.909) (width 0.2) (layer "B.Cu") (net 14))
 (segment (start 131.8843 122.6228) (end 131.8843 125.6112) (width 0.2) (layer "B.Cu") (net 20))
 (segment (start 131.8957 122.6114) (end 131.8843 122.6228) (width 0.2) (layer "B.Cu") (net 20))
 (segment (start 133.5118 122.6114) (end 131.8957 122.6114) (width 0.2) (layer "B.Cu") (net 20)))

